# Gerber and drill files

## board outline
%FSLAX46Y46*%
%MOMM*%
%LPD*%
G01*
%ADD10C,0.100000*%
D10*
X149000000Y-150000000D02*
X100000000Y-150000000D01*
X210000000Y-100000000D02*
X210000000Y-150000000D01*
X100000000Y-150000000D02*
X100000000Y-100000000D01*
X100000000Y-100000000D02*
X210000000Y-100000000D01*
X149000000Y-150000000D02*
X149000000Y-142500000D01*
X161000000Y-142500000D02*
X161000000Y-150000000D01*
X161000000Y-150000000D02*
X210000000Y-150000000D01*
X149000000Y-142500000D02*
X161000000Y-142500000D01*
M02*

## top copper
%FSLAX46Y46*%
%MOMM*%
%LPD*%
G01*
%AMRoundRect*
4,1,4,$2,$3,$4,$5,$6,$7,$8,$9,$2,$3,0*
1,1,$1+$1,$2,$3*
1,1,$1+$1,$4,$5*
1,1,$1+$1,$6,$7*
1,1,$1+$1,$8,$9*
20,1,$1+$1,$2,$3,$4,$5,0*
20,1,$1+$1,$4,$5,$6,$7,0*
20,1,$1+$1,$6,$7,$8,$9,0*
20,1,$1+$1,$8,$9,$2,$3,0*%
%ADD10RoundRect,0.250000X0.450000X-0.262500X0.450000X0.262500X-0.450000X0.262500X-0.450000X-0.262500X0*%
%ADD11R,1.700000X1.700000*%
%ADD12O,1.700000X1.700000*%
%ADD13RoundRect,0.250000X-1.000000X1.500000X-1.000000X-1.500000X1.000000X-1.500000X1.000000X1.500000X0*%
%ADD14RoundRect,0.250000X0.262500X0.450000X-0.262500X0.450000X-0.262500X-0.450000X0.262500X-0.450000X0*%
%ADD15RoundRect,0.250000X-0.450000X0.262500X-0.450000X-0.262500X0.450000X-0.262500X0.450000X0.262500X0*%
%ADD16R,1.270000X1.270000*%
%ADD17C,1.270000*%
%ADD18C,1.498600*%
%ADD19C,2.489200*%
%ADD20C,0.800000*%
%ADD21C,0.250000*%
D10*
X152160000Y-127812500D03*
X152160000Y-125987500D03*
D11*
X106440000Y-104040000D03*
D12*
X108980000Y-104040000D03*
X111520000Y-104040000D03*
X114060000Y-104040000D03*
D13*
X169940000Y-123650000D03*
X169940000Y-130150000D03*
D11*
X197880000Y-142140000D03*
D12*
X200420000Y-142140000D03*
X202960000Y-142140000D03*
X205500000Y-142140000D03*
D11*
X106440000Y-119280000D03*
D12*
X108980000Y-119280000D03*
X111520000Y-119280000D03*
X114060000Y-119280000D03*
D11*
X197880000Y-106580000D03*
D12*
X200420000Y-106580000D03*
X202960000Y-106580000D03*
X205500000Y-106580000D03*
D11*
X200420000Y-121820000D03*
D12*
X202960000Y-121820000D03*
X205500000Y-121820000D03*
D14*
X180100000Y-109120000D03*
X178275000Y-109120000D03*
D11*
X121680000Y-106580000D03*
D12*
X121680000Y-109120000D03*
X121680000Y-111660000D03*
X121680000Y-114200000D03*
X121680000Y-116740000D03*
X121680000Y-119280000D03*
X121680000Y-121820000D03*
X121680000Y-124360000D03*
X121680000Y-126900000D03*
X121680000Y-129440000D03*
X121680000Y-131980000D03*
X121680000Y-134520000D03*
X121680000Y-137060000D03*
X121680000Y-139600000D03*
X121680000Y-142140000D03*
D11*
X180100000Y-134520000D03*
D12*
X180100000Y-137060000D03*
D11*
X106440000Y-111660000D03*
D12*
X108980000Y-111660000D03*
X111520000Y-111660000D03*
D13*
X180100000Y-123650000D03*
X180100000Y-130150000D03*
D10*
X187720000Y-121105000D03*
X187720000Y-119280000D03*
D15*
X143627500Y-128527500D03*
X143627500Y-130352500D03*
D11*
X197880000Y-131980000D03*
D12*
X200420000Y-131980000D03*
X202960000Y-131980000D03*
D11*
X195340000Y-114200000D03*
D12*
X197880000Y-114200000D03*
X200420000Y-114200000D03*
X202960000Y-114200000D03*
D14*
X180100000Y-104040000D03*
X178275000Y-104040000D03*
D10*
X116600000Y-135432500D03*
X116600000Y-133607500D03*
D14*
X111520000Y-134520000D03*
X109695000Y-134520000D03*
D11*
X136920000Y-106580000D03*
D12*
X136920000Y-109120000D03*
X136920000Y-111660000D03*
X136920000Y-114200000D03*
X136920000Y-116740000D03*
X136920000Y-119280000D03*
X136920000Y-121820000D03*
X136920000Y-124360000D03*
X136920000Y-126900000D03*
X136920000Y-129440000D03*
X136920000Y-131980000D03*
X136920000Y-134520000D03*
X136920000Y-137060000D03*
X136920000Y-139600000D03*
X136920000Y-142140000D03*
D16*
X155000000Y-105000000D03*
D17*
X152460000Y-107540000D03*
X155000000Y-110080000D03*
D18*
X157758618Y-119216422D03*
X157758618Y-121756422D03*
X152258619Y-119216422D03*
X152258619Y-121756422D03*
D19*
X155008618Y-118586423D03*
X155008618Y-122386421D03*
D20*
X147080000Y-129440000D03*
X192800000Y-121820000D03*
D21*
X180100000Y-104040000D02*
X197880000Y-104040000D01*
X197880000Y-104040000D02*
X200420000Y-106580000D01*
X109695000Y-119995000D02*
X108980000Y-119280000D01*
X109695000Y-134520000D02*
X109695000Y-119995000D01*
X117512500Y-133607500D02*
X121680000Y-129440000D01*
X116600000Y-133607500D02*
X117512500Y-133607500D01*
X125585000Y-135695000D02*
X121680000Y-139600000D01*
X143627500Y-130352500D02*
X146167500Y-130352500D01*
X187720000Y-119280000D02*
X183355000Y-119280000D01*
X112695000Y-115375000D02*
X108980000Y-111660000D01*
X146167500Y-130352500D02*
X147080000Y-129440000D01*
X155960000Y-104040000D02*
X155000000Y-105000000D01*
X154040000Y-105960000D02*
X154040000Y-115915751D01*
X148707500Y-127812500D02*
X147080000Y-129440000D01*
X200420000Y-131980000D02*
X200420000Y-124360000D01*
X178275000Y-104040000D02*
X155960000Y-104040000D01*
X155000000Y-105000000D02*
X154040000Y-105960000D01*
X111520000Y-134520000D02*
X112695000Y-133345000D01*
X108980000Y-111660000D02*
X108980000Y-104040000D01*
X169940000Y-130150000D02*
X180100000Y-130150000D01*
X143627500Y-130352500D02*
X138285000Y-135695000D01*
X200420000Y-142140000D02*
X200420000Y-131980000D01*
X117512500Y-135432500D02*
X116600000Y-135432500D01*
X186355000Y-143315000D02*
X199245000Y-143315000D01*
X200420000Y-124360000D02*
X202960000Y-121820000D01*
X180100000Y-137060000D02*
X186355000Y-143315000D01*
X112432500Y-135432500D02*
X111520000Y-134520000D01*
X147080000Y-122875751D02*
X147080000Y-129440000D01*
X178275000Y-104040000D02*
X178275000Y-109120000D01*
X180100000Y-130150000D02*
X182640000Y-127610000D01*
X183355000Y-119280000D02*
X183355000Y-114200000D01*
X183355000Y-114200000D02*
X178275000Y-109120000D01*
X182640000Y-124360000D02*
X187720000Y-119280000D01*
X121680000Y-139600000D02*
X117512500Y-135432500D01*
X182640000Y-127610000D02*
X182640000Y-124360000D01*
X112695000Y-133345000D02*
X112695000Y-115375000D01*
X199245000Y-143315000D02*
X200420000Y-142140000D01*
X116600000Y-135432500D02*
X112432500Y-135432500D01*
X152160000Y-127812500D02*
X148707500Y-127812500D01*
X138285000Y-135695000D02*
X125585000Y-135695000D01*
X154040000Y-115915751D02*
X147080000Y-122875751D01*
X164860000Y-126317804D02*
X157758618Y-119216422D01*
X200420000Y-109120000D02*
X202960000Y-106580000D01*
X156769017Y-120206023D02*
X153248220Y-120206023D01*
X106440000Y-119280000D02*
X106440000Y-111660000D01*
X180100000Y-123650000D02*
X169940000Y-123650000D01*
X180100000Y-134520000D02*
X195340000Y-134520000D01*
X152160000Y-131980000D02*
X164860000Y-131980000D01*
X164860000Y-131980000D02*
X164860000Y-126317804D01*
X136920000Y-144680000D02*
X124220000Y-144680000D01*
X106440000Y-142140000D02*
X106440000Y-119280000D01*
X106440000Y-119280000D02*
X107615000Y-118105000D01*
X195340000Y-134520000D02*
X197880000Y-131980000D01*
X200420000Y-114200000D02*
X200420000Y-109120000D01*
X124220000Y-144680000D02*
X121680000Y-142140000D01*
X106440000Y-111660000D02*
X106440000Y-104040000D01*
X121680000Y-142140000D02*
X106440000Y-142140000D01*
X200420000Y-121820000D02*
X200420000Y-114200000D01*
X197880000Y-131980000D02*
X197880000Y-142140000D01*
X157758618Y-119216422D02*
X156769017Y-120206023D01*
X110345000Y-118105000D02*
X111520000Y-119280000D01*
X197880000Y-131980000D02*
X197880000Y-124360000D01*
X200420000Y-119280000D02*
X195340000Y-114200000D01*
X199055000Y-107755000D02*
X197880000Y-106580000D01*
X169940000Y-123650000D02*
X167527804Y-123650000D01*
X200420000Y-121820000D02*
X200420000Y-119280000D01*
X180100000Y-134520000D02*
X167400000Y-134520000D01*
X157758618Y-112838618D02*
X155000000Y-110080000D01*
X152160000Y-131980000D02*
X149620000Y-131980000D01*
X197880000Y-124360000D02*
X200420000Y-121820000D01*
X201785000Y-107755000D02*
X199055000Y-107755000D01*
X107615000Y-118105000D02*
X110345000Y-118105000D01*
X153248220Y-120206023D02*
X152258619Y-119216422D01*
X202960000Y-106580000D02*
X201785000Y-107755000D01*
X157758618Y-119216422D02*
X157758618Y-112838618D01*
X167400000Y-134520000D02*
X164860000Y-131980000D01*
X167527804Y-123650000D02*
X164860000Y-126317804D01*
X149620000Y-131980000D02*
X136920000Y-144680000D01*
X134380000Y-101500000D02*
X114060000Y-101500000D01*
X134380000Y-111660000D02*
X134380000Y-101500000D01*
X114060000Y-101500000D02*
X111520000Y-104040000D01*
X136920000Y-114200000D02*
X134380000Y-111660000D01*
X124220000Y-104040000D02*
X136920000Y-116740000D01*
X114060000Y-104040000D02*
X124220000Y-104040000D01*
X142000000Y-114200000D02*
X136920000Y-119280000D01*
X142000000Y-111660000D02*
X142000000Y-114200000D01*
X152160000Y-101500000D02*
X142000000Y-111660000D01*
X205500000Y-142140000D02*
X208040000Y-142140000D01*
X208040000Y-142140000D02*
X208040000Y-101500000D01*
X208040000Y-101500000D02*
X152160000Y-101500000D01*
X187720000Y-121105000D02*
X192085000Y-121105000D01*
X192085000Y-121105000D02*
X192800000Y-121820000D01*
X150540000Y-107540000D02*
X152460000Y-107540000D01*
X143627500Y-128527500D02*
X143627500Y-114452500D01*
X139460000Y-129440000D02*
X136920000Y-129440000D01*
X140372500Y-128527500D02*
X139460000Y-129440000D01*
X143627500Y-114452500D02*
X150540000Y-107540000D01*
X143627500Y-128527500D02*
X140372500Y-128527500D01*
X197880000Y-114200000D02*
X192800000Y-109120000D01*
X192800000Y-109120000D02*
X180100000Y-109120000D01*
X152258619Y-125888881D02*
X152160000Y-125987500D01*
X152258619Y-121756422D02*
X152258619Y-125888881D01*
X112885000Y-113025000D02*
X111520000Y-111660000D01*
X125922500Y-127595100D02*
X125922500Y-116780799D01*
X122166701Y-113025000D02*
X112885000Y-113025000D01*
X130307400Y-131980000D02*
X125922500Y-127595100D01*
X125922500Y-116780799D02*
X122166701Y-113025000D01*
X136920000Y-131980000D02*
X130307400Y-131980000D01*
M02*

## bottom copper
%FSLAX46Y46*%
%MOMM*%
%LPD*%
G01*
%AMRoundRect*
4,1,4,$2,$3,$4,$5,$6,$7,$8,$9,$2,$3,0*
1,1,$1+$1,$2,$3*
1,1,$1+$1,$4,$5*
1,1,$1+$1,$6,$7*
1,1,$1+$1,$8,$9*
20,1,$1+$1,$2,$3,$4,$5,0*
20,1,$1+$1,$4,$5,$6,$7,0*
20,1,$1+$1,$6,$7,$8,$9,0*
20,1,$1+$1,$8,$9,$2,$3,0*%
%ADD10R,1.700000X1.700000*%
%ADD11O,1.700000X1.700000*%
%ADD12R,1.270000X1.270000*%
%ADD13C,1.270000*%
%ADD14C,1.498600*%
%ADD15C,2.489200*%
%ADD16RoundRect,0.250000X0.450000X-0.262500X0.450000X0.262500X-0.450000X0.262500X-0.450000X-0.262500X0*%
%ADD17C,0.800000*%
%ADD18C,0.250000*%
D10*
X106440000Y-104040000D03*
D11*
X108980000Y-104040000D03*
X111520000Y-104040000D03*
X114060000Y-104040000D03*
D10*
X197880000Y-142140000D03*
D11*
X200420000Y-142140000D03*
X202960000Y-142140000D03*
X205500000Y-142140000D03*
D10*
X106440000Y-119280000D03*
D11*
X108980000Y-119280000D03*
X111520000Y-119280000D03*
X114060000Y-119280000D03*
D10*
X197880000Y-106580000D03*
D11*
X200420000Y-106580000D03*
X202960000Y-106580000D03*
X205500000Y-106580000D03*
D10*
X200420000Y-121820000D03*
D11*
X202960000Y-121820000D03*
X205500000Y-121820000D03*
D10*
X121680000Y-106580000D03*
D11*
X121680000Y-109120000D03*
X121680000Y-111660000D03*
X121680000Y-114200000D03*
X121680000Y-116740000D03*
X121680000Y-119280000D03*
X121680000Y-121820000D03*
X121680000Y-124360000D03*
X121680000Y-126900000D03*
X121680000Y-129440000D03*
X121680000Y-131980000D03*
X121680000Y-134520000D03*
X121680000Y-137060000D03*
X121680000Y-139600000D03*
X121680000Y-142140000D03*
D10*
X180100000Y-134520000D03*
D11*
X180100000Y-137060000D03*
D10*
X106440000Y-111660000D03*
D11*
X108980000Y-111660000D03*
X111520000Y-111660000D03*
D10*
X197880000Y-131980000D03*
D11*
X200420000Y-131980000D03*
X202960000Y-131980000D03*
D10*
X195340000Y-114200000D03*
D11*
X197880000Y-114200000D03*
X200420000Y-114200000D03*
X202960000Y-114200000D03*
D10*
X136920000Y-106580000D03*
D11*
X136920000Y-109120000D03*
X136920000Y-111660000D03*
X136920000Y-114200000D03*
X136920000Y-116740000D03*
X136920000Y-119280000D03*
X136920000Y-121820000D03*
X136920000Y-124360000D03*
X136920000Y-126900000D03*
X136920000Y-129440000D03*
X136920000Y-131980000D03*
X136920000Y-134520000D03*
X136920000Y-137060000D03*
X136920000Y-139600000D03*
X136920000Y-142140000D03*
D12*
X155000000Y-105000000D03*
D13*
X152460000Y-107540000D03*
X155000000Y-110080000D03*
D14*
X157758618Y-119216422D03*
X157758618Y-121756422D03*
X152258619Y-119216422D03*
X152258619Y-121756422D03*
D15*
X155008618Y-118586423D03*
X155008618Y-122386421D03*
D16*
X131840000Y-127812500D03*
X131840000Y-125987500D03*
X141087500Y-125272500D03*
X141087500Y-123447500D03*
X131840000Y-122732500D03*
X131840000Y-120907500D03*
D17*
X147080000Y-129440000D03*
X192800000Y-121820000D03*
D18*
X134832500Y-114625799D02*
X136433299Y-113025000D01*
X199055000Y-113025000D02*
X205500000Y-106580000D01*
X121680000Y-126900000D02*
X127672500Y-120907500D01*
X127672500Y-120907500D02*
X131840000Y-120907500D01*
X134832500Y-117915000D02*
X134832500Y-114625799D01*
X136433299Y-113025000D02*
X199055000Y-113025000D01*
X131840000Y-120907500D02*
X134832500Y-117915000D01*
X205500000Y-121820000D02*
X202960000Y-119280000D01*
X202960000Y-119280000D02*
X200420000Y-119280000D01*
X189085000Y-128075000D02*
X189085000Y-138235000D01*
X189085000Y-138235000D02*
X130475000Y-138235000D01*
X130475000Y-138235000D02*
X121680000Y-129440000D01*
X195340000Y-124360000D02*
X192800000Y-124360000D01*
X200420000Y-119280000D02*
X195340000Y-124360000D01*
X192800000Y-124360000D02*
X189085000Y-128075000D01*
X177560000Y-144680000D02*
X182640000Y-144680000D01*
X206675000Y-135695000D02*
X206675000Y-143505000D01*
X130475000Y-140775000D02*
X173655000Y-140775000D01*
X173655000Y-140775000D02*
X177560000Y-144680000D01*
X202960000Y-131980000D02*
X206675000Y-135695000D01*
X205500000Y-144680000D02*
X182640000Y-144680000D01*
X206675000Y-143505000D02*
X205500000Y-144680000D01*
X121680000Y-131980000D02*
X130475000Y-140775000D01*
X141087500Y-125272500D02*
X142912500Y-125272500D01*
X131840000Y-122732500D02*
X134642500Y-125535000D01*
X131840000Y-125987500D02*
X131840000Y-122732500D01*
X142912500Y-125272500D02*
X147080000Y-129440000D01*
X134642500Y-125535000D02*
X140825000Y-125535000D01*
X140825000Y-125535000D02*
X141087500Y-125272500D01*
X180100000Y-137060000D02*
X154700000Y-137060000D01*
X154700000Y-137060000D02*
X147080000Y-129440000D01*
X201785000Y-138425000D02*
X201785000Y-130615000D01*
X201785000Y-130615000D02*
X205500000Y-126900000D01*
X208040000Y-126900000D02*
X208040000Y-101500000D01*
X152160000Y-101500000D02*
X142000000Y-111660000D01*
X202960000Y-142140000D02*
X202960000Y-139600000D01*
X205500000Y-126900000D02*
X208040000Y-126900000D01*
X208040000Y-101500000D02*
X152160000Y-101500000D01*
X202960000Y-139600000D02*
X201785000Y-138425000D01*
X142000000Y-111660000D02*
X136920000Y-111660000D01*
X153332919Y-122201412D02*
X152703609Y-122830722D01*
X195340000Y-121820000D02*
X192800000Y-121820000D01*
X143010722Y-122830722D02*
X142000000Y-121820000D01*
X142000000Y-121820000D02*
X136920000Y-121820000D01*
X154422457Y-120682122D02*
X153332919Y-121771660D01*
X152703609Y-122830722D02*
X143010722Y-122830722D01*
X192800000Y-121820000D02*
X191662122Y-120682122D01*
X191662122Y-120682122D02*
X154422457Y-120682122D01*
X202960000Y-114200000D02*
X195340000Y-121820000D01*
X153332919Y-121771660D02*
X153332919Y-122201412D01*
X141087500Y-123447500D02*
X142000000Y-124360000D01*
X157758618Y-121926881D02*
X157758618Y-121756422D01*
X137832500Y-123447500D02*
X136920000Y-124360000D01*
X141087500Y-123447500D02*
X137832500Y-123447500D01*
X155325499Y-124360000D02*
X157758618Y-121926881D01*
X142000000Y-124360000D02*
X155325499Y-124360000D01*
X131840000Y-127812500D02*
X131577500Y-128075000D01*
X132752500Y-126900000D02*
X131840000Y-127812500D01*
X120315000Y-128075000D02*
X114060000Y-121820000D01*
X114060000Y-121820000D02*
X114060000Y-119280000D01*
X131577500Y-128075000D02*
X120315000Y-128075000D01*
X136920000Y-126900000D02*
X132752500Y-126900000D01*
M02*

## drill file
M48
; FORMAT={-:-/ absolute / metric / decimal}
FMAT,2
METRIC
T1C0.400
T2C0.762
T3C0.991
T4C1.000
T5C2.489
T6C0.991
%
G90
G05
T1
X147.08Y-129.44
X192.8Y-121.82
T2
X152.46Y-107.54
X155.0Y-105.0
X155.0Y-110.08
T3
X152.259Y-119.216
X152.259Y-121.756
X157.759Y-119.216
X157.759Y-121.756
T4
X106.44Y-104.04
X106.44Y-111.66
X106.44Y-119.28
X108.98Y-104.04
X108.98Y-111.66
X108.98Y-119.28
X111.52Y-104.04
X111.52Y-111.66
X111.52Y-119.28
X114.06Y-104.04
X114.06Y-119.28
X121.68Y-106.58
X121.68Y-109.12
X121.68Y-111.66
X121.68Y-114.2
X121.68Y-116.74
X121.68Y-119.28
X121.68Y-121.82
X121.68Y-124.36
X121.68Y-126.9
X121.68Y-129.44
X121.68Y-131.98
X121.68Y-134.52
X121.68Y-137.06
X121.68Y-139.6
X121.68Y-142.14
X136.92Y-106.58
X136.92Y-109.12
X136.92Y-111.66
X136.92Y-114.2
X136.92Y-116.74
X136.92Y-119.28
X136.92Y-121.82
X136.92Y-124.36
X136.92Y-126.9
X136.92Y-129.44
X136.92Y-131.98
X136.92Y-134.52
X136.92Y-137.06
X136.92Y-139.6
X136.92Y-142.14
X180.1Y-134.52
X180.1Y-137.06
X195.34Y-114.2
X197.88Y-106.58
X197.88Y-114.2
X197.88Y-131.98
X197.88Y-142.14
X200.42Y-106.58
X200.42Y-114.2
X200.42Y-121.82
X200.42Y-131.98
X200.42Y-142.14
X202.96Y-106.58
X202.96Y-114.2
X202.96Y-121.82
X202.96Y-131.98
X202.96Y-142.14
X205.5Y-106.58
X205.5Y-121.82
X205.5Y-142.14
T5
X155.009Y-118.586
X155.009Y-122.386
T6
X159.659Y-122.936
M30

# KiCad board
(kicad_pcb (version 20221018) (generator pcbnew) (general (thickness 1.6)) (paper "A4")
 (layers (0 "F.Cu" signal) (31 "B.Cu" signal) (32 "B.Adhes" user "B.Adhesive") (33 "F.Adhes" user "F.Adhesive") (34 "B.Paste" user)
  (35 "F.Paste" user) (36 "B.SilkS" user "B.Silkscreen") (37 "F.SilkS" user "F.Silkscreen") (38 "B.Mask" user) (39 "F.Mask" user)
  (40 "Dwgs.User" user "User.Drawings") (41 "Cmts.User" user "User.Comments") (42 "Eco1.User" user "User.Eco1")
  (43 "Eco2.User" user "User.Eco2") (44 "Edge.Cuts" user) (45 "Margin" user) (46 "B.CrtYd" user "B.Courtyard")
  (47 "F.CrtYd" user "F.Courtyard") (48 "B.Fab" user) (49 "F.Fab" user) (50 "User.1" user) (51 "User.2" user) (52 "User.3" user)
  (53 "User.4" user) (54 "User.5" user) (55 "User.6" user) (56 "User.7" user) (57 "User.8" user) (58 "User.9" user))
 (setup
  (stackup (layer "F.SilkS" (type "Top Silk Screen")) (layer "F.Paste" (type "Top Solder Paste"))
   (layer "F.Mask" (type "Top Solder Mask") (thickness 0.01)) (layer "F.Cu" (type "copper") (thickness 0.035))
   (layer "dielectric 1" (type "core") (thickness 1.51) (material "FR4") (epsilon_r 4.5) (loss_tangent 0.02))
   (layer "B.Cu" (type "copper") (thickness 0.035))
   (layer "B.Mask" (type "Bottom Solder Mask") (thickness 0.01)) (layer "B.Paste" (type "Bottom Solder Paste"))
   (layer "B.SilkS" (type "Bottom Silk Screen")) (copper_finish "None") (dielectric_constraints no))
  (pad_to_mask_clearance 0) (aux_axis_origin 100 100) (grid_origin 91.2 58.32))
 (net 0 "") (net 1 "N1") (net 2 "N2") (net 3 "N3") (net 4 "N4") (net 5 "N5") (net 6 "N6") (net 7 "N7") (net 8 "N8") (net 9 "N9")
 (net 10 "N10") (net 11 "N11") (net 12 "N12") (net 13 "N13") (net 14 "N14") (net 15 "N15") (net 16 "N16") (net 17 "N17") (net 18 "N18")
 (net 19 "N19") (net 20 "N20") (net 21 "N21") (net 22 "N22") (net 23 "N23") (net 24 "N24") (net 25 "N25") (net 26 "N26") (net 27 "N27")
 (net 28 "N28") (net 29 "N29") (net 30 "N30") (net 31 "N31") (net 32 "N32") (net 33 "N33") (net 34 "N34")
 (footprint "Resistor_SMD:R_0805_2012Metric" (layer "F.Cu") (at 152.16 126.9 90)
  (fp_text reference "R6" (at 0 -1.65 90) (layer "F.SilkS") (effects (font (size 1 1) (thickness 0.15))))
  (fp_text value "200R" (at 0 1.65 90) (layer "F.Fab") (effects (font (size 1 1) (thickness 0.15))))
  (pad "1" smd roundrect (at -0.9125 0 90) (size 1.025 1.4) (layers "F.Cu" "F.Paste" "F.Mask") (roundrect_rratio 0.243902) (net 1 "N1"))
  (pad "2" smd roundrect (at 0.9125 0 90) (size 1.025 1.4) (layers "F.Cu" "F.Paste" "F.Mask") (roundrect_rratio 0.243902) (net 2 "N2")))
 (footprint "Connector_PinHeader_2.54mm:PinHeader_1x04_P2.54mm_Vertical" (layer "F.Cu") (at 106.44 104.04 90)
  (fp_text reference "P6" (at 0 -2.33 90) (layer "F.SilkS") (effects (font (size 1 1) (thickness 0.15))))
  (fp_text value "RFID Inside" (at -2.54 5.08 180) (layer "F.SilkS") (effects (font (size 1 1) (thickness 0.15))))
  (pad "1" thru_hole rect (at 0 0 90) (size 1.7 1.7) (drill 1) (layers "*.Cu" "*.Mask") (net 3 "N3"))
  (pad "2" thru_hole oval (at 0 2.54 90) (size 1.7 1.7) (drill 1) (layers "*.Cu" "*.Mask") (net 1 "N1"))
  (pad "3" thru_hole oval (at 0 5.08 90) (size 1.7 1.7) (drill 1) (layers "*.Cu" "*.Mask") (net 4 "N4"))
  (pad "4" thru_hole oval (at 0 7.62 90) (size 1.7 1.7) (drill 1) (layers "*.Cu" "*.Mask") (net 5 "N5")))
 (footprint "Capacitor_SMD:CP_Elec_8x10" (layer "F.Cu") (at 169.94 126.9 -90)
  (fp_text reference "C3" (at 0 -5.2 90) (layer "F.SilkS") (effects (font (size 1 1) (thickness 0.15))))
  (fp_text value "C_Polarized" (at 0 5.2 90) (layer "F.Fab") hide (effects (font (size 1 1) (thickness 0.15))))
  (pad "1" smd roundrect (at -3.25 0 270) (size 3.5 2.5) (layers "F.Cu" "F.Paste" "F.Mask") (roundrect_rratio 0.1) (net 3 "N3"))
  (pad "2" smd roundrect (at 3.25 0 270) (size 3.5 2.5) (layers "F.Cu" "F.Paste" "F.Mask") (roundrect_rratio 0.1) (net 1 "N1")))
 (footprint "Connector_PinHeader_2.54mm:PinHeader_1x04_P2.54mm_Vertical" (layer "F.Cu") (at 197.88 142.14 90)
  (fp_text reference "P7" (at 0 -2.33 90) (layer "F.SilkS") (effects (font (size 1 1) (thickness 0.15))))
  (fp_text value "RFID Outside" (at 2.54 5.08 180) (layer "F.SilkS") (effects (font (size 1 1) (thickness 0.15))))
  (pad "1" thru_hole rect (at 0 0 90) (size 1.7 1.7) (drill 1) (layers "*.Cu" "*.Mask") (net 3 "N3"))
  (pad "2" thru_hole oval (at 0 2.54 90) (size 1.7 1.7) (drill 1) (layers "*.Cu" "*.Mask") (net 1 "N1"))
  (pad "3" thru_hole oval (at 0 5.08 90) (size 1.7 1.7) (drill 1) (layers "*.Cu" "*.Mask") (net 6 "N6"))
  (pad "4" thru_hole oval (at 0 7.62 90) (size 1.7 1.7) (drill 1) (layers "*.Cu" "*.Mask") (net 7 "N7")))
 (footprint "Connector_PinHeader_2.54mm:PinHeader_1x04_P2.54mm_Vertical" (layer "F.Cu") (at 106.44 119.28 90)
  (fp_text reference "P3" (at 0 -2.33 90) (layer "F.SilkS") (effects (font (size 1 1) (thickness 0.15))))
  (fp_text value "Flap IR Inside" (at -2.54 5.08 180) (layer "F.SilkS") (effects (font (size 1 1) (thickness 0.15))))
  (pad "1" thru_hole rect (at 0 0 90) (size 1.7 1.7) (drill 1) (layers "*.Cu" "*.Mask") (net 3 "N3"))
  (pad "2" thru_hole oval (at 0 2.54 90) (size 1.7 1.7) (drill 1) (layers "*.Cu" "*.Mask") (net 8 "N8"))
  (pad "3" thru_hole oval (at 0 5.08 90) (size 1.7 1.7) (drill 1) (layers "*.Cu" "*.Mask") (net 3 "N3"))
  (pad "4" thru_hole oval (at 0 7.62 90) (size 1.7 1.7) (drill 1) (layers "*.Cu" "*.Mask") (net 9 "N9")))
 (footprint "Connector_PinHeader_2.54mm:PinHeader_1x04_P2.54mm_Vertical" (layer "F.Cu") (at 197.88 106.58 90)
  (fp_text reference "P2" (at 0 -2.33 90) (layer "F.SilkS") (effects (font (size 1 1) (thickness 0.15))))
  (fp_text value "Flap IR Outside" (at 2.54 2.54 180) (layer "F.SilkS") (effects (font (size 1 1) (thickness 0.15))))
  (pad "1" thru_hole rect (at 0 0 90) (size 1.7 1.7) (drill 1) (layers "*.Cu" "*.Mask") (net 3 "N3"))
  (pad "2" thru_hole oval (at 0 2.54 90) (size 1.7 1.7) (drill 1) (layers "*.Cu" "*.Mask") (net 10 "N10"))
  (pad "3" thru_hole oval (at 0 5.08 90) (size 1.7 1.7) (drill 1) (layers "*.Cu" "*.Mask") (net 3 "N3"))
  (pad "4" thru_hole oval (at 0 7.62 90) (size 1.7 1.7) (drill 1) (layers "*.Cu" "*.Mask") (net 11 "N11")))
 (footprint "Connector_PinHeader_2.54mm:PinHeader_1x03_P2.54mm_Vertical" (layer "F.Cu") (at 200.42 121.82 90)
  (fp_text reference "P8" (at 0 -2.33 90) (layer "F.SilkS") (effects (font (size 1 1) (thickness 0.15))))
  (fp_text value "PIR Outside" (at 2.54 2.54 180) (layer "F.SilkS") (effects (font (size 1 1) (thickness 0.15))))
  (pad "1" thru_hole rect (at 0 0 90) (size 1.7 1.7) (drill 1) (layers "*.Cu" "*.Mask") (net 3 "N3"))
  (pad "2" thru_hole oval (at 0 2.54 90) (size 1.7 1.7) (drill 1) (layers "*.Cu" "*.Mask") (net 1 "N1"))
  (pad "3" thru_hole oval (at 0 5.08 90) (size 1.7 1.7) (drill 1) (layers "*.Cu" "*.Mask") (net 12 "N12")))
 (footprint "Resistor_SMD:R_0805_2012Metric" (layer "F.Cu") (at 179.1875 109.12 180)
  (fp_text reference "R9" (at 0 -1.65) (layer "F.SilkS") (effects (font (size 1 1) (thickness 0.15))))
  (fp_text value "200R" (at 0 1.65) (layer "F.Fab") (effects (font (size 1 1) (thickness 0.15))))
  (pad "1" smd roundrect (at -0.9125 0 180) (size 1.025 1.4) (layers "F.Cu" "F.Paste" "F.Mask") (roundrect_rratio 0.243902) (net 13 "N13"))
  (pad "2" smd roundrect (at 0.9125 0 180) (size 1.025 1.4) (layers "F.Cu" "F.Paste" "F.Mask") (roundrect_rratio 0.243902) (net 1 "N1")))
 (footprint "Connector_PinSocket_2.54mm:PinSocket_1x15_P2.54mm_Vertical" (layer "F.Cu") (at 121.68 106.58)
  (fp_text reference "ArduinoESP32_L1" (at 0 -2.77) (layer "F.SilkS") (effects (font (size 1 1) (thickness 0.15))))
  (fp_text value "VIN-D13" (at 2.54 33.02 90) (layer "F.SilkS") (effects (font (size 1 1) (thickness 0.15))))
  (pad "1" thru_hole rect (at 0 0) (size 1.7 1.7) (drill 1) (layers "*.Cu" "*.Mask") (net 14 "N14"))
  (pad "2" thru_hole oval (at 0 2.54) (size 1.7 1.7) (drill 1) (layers "*.Cu" "*.Mask") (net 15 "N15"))
  (pad "3" thru_hole oval (at 0 5.08) (size 1.7 1.7) (drill 1) (layers "*.Cu" "*.Mask") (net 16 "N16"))
  (pad "4" thru_hole oval (at 0 7.62) (size 1.7 1.7) (drill 1) (layers "*.Cu" "*.Mask") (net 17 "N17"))
  (pad "5" thru_hole oval (at 0 10.16) (size 1.7 1.7) (drill 1) (layers "*.Cu" "*.Mask") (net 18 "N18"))
  (pad "6" thru_hole oval (at 0 12.7) (size 1.7 1.7) (drill 1) (layers "*.Cu" "*.Mask") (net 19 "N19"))
  (pad "7" thru_hole oval (at 0 15.24) (size 1.7 1.7) (drill 1) (layers "*.Cu" "*.Mask") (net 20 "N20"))
  (pad "8" thru_hole oval (at 0 17.78) (size 1.7 1.7) (drill 1) (layers "*.Cu" "*.Mask") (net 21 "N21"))
  (pad "9" thru_hole oval (at 0 20.32) (size 1.7 1.7) (drill 1) (layers "*.Cu" "*.Mask") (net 11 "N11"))
  (pad "10" thru_hole oval (at 0 22.86) (size 1.7 1.7) (drill 1) (layers "*.Cu" "*.Mask") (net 12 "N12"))
  (pad "11" thru_hole oval (at 0 25.4) (size 1.7 1.7) (drill 1) (layers "*.Cu" "*.Mask") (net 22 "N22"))
  (pad "12" thru_hole oval (at 0 27.94) (size 1.7 1.7) (drill 1) (layers "*.Cu" "*.Mask") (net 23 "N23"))
  (pad "13" thru_hole oval (at 0 30.48) (size 1.7 1.7) (drill 1) (layers "*.Cu" "*.Mask") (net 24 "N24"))
  (pad "14" thru_hole oval (at 0 33.02) (size 1.7 1.7) (drill 1) (layers "*.Cu" "*.Mask") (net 1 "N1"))
  (pad "15" thru_hole oval (at 0 35.56) (size 1.7 1.7) (drill 1) (layers "*.Cu" "*.Mask") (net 3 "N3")))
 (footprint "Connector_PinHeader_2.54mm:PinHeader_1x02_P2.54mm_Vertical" (layer "F.Cu") (at 180.1 134.52)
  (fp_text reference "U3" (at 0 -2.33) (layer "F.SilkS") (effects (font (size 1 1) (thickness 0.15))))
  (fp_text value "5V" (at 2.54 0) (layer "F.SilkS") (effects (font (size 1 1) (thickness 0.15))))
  (pad "1" thru_hole rect (at 0 0) (size 1.7 1.7) (drill 1) (layers "*.Cu" "*.Mask") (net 3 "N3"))
  (pad "2" thru_hole oval (at 0 2.54) (size 1.7 1.7) (drill 1) (layers "*.Cu" "*.Mask") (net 1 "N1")))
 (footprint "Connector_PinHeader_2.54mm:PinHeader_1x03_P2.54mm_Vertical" (layer "F.Cu") (at 106.44 111.66 90)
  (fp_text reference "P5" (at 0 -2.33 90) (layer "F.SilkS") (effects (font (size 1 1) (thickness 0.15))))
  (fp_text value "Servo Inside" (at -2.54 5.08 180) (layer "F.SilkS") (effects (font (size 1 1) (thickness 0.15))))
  (pad "1" thru_hole rect (at 0 0 90) (size 1.7 1.7) (drill 1) (layers "*.Cu" "*.Mask") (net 3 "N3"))
  (pad "2" thru_hole oval (at 0 2.54 90) (size 1.7 1.7) (drill 1) (layers "*.Cu" "*.Mask") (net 1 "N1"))
  (pad "3" thru_hole oval (at 0 5.08 90) (size 1.7 1.7) (drill 1) (layers "*.Cu" "*.Mask") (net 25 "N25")))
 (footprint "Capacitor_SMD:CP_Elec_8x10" (layer "F.Cu") (at 180.1 126.9 -90)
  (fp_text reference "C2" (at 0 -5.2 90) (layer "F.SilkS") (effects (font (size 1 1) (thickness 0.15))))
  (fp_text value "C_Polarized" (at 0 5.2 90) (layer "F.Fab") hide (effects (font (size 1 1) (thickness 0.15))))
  (pad "1" smd roundrect (at -3.25 0 270) (size 3.5 2.5) (layers "F.Cu" "F.Paste" "F.Mask") (roundrect_rratio 0.1) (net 3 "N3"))
  (pad "2" smd roundrect (at 3.25 0 270) (size 3.5 2.5) (layers "F.Cu" "F.Paste" "F.Mask") (roundrect_rratio 0.1) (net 1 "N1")))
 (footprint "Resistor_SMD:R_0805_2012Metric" (layer "F.Cu") (at 187.72 120.1925 90)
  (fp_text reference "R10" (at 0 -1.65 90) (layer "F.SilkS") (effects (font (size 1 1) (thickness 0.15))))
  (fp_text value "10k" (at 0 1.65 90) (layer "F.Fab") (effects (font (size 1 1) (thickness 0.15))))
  (pad "1" smd roundrect (at -0.9125 0 90) (size 1.025 1.4) (layers "F.Cu" "F.Paste" "F.Mask") (roundrect_rratio 0.243902) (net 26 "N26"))
  (pad "2" smd roundrect (at 0.9125 0 90) (size 1.025 1.4) (layers "F.Cu" "F.Paste" "F.Mask") (roundrect_rratio 0.243902) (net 1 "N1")))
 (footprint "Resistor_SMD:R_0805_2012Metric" (layer "F.Cu") (at 143.6275 129.44 -90)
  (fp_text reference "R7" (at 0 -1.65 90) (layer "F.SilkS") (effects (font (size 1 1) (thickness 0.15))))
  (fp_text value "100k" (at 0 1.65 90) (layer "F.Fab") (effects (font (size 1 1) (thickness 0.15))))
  (pad "1" smd roundrect (at -0.9125 0 270) (size 1.025 1.4) (layers "F.Cu" "F.Paste" "F.Mask") (roundrect_rratio 0.243902) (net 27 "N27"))
  (pad "2" smd roundrect (at 0.9125 0 270) (size 1.025 1.4) (layers "F.Cu" "F.Paste" "F.Mask") (roundrect_rratio 0.243902) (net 1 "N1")))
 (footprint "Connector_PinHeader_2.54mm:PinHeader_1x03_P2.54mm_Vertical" (layer "F.Cu") (at 197.88 131.98 90)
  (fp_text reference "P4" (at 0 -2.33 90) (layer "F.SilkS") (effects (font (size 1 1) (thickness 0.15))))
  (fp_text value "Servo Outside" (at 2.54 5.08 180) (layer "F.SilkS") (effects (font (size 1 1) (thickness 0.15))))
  (pad "1" thru_hole rect (at 0 0 90) (size 1.7 1.7) (drill 1) (layers "*.Cu" "*.Mask") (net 3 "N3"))
  (pad "2" thru_hole oval (at 0 2.54 90) (size 1.7 1.7) (drill 1) (layers "*.Cu" "*.Mask") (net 1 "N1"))
  (pad "3" thru_hole oval (at 0 5.08 90) (size 1.7 1.7) (drill 1) (layers "*.Cu" "*.Mask") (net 22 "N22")))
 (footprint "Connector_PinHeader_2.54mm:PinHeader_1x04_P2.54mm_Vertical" (layer "F.Cu") (at 195.34 114.2 90)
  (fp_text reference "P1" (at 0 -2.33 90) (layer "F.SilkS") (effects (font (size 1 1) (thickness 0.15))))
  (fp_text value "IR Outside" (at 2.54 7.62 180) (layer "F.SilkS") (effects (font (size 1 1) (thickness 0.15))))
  (pad "1" thru_hole rect (at 0 0 90) (size 1.7 1.7) (drill 1) (layers "*.Cu" "*.Mask") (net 3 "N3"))
  (pad "2" thru_hole oval (at 0 2.54 90) (size 1.7 1.7) (drill 1) (layers "*.Cu" "*.Mask") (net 13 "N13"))
  (pad "3" thru_hole oval (at 0 5.08 90) (size 1.7 1.7) (drill 1) (layers "*.Cu" "*.Mask") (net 3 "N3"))
  (pad "4" thru_hole oval (at 0 7.62 90) (size 1.7 1.7) (drill 1) (layers "*.Cu" "*.Mask") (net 26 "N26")))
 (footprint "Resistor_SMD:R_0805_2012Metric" (layer "F.Cu") (at 179.1875 104.04 180)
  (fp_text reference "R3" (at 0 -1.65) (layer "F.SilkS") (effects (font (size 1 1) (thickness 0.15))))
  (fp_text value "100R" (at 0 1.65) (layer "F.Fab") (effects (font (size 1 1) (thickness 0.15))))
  (pad "1" smd roundrect (at -0.9125 0 180) (size 1.025 1.4) (layers "F.Cu" "F.Paste" "F.Mask") (roundrect_rratio 0.243902) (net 10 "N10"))
  (pad "2" smd roundrect (at 0.9125 0 180) (size 1.025 1.4) (layers "F.Cu" "F.Paste" "F.Mask") (roundrect_rratio 0.243902) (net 1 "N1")))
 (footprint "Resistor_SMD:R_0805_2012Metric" (layer "F.Cu") (at 116.6 134.52 90)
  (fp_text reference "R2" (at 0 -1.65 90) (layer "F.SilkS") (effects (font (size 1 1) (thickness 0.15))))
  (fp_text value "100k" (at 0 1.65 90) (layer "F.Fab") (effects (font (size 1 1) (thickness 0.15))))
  (pad "1" smd roundrect (at -0.9125 0 90) (size 1.025 1.4) (layers "F.Cu" "F.Paste" "F.Mask") (roundrect_rratio 0.243902) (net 1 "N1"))
  (pad "2" smd roundrect (at 0.9125 0 90) (size 1.025 1.4) (layers "F.Cu" "F.Paste" "F.Mask") (roundrect_rratio 0.243902) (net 12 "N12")))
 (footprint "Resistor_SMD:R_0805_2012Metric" (layer "F.Cu") (at 110.6075 134.52 180)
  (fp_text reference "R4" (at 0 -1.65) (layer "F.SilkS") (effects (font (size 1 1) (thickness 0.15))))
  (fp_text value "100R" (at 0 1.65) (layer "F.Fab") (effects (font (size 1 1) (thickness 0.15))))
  (pad "1" smd roundrect (at -0.9125 0 180) (size 1.025 1.4) (layers "F.Cu" "F.Paste" "F.Mask") (roundrect_rratio 0.243902) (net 1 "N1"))
  (pad "2" smd roundrect (at 0.9125 0 180) (size 1.025 1.4) (layers "F.Cu" "F.Paste" "F.Mask") (roundrect_rratio 0.243902) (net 8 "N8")))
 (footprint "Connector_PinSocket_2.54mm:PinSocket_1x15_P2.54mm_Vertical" (layer "F.Cu") (at 136.92 106.58)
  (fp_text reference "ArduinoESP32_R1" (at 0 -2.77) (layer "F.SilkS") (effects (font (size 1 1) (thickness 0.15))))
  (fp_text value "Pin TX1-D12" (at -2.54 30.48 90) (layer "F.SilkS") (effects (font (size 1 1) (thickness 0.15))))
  (pad "1" thru_hole rect (at 0 0) (size 1.7 1.7) (drill 1) (layers "*.Cu" "*.Mask") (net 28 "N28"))
  (pad "2" thru_hole oval (at 0 2.54) (size 1.7 1.7) (drill 1) (layers "*.Cu" "*.Mask") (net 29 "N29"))
  (pad "3" thru_hole oval (at 0 5.08) (size 1.7 1.7) (drill 1) (layers "*.Cu" "*.Mask") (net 6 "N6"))
  (pad "4" thru_hole oval (at 0 7.62) (size 1.7 1.7) (drill 1) (layers "*.Cu" "*.Mask") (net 4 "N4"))
  (pad "5" thru_hole oval (at 0 10.16) (size 1.7 1.7) (drill 1) (layers "*.Cu" "*.Mask") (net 5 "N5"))
  (pad "6" thru_hole oval (at 0 12.7) (size 1.7 1.7) (drill 1) (layers "*.Cu" "*.Mask") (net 7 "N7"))
  (pad "7" thru_hole oval (at 0 15.24) (size 1.7 1.7) (drill 1) (layers "*.Cu" "*.Mask") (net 26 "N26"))
  (pad "8" thru_hole oval (at 0 17.78) (size 1.7 1.7) (drill 1) (layers "*.Cu" "*.Mask") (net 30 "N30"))
  (pad "9" thru_hole oval (at 0 20.32) (size 1.7 1.7) (drill 1) (layers "*.Cu" "*.Mask") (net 9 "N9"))
  (pad "10" thru_hole oval (at 0 22.86) (size 1.7 1.7) (drill 1) (layers "*.Cu" "*.Mask") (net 27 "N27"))
  (pad "11" thru_hole oval (at 0 25.4) (size 1.7 1.7) (drill 1) (layers "*.Cu" "*.Mask") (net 25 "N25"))
  (pad "12" thru_hole oval (at 0 27.94) (size 1.7 1.7) (drill 1) (layers "*.Cu" "*.Mask") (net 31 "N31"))
  (pad "13" thru_hole oval (at 0 30.48) (size 1.7 1.7) (drill 1) (layers "*.Cu" "*.Mask") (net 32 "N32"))
  (pad "14" thru_hole oval (at 0 33.02) (size 1.7 1.7) (drill 1) (layers "*.Cu" "*.Mask") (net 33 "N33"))
  (pad "15" thru_hole oval (at 0 35.56) (size 1.7 1.7) (drill 1) (layers "*.Cu" "*.Mask") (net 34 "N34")))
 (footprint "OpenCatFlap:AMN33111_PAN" (layer "B.Cu") (at 155 105 180)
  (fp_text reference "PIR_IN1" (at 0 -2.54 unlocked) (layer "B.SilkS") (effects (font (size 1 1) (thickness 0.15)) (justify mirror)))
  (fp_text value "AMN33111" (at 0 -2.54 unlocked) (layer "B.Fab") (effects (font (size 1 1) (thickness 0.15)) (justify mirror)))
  (pad "1" thru_hole rect (at 0 0 180) (size 1.27 1.27) (drill 0.762) (layers "*.Cu" "*.Mask") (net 1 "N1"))
  (pad "2" thru_hole circle (at 2.54 -2.54 90) (size 1.27 1.27) (drill 0.762) (layers "*.Cu" "*.Mask") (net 27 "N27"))
  (pad "3" thru_hole circle (at 0 -5.08 180) (size 1.27 1.27) (drill 0.762) (layers "*.Cu" "*.Mask") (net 3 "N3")))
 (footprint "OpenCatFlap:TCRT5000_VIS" (layer "B.Cu") (at 157.758618 119.216422 180)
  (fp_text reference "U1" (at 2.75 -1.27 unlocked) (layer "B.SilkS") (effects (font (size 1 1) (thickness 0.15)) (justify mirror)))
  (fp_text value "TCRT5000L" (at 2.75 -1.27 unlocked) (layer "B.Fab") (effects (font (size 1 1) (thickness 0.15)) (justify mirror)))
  (pad "" np_thru_hole circle (at -1.900001 -3.72 180) (size 0.9906 0.9906) (drill 0.9906) (layers "*.Cu" "*.Mask"))
  (pad "1" thru_hole circle (at 0 0 180) (size 1.4986 1.4986) (drill 0.9906) (layers "*.Cu" "*.Mask") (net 3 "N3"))
  (pad "2" thru_hole circle (at 0 -2.54 180) (size 1.4986 1.4986) (drill 0.9906) (layers "*.Cu" "*.Mask") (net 30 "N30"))
  (pad "3" thru_hole circle (at 5.499999 0 180) (size 1.4986 1.4986) (drill 0.9906) (layers "*.Cu" "*.Mask") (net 3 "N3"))
  (pad "4" thru_hole circle (at 5.499999 -2.54 180) (size 1.4986 1.4986) (drill 0.9906) (layers "*.Cu" "*.Mask") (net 2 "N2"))
  (pad "5" thru_hole circle (at 2.75 0.629999 180) (size 2.4892 2.4892) (drill 2.4892) (layers "*.Cu" "*.Mask"))
  (pad "6" thru_hole circle (at 2.75 -3.169999 180) (size 2.4892 2.4892) (drill 2.4892) (layers "*.Cu" "*.Mask")))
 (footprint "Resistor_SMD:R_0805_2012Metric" (layer "B.Cu") (at 131.84 126.9 90)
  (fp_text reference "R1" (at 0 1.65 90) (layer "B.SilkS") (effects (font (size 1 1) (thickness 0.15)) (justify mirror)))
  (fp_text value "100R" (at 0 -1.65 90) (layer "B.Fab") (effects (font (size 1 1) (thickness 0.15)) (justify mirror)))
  (pad "1" smd roundrect (at -0.9125 0 90) (size 1.025 1.4) (layers "B.Cu" "B.Paste" "B.Mask") (roundrect_rratio 0.243902) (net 9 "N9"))
  (pad "2" smd roundrect (at 0.9125 0 90) (size 1.025 1.4) (layers "B.Cu" "B.Paste" "B.Mask") (roundrect_rratio 0.243902) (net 1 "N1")))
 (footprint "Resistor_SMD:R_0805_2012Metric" (layer "B.Cu") (at 141.0875 124.36 90)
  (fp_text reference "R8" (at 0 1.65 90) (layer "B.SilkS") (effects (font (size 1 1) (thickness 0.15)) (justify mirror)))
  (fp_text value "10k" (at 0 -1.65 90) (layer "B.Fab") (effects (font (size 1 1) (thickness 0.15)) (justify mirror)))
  (pad "1" smd roundrect (at -0.9125 0 90) (size 1.025 1.4) (layers "B.Cu" "B.Paste" "B.Mask") (roundrect_rratio 0.243902) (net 1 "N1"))
  (pad "2" smd roundrect (at 0.9125 0 90) (size 1.025 1.4) (layers "B.Cu" "B.Paste" "B.Mask") (roundrect_rratio 0.243902) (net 30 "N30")))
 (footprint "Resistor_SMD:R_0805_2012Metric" (layer "B.Cu") (at 131.84 121.82 90)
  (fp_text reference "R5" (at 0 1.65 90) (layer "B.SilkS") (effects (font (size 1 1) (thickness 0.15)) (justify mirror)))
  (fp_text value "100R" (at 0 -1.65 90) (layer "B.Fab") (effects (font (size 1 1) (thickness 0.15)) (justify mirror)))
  (pad "1" smd roundrect (at -0.9125 0 90) (size 1.025 1.4) (layers "B.Cu" "B.Paste" "B.Mask") (roundrect_rratio 0.243902) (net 1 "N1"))
  (pad "2" smd roundrect (at 0.9125 0 90) (size 1.025 1.4) (layers "B.Cu" "B.Paste" "B.Mask") (roundrect_rratio 0.243902) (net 11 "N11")))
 (gr_line (start 149 150) (end 100 150) (stroke (width 0.1) (type default)) (layer "Edge.Cuts"))
 (gr_line locked (start 210 100) (end 210 150) (stroke (width 0.1) (type default)) (layer "Edge.Cuts"))
 (gr_line locked (start 100 150) (end 100 100) (stroke (width 0.1) (type default)) (layer "Edge.Cuts"))
 (gr_line locked (start 100 100) (end 210 100) (stroke (width 0.1) (type default)) (layer "Edge.Cuts"))
 (gr_line (start 149 150) (end 149 142.5) (stroke (width 0.1) (type default)) (layer "Edge.Cuts"))
 (gr_line (start 161 142.5) (end 161 150) (stroke (width 0.1) (type default)) (layer "Edge.Cuts"))
 (gr_line (start 161 150) (end 210 150) (stroke (width 0.1) (type default)) (layer "Edge.Cuts"))
 (gr_line (start 149 142.5) (end 161 142.5) (stroke (width 0.1) (type default)) (layer "Edge.Cuts"))
 (segment (start 180.1 104.04) (end 197.88 104.04) (width 0.25) (layer "F.Cu") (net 10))
 (segment (start 197.88 104.04) (end 200.42 106.58) (width 0.25) (layer "F.Cu") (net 10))
 (segment (start 109.695 119.995) (end 108.98 119.28) (width 0.25) (layer "F.Cu") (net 8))
 (segment (start 109.695 134.52) (end 109.695 119.995) (width 0.25) (layer "F.Cu") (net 8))
 (segment (start 134.8325 114.625799) (end 136.433299 113.025) (width 0.25) (layer "B.Cu") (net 11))
 (segment (start 199.055 113.025) (end 205.5 106.58) (width 0.25) (layer "B.Cu") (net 11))
 (segment (start 121.68 126.9) (end 127.6725 120.9075) (width 0.25) (layer "B.Cu") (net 11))
 (segment (start 127.6725 120.9075) (end 131.84 120.9075) (width 0.25) (layer "B.Cu") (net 11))
 (segment (start 134.8325 117.915) (end 134.8325 114.625799) (width 0.25) (layer "B.Cu") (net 11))
 (segment (start 136.433299 113.025) (end 199.055 113.025) (width 0.25) (layer "B.Cu") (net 11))
 (segment (start 131.84 120.9075) (end 134.8325 117.915) (width 0.25) (layer "B.Cu") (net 11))
 (segment (start 117.5125 133.6075) (end 121.68 129.44) (width 0.25) (layer "F.Cu") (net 12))
 (segment (start 116.6 133.6075) (end 117.5125 133.6075) (width 0.25) (layer "F.Cu") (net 12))
 (segment (start 205.5 121.82) (end 202.96 119.28) (width 0.25) (layer "B.Cu") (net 12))
 (segment (start 202.96 119.28) (end 200.42 119.28) (width 0.25) (layer "B.Cu") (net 12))
 (segment (start 189.085 128.075) (end 189.085 138.235) (width 0.25) (layer "B.Cu") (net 12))
 (segment (start 189.085 138.235) (end 130.475 138.235) (width 0.25) (layer "B.Cu") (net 12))
 (segment (start 130.475 138.235) (end 121.68 129.44) (width 0.25) (layer "B.Cu") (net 12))
 (segment (start 195.34 124.36) (end 192.8 124.36) (width 0.25) (layer "B.Cu") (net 12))
 (segment (start 200.42 119.28) (end 195.34 124.36) (width 0.25) (layer "B.Cu") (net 12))
 (segment (start 192.8 124.36) (end 189.085 128.075) (width 0.25) (layer "B.Cu") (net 12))
 (segment (start 177.56 144.68) (end 182.64 144.68) (width 0.25) (layer "B.Cu") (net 22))
 (segment (start 206.675 135.695) (end 206.675 143.505) (width 0.25) (layer "B.Cu") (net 22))
 (segment (start 130.475 140.775) (end 173.655 140.775) (width 0.25) (layer "B.Cu") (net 22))
 (segment (start 173.655 140.775) (end 177.56 144.68) (width 0.25) (layer "B.Cu") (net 22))
 (segment (start 202.96 131.98) (end 206.675 135.695) (width 0.25) (layer "B.Cu") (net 22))
 (segment (start 205.5 144.68) (end 182.64 144.68) (width 0.25) (layer "B.Cu") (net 22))
 (segment (start 206.675 143.505) (end 205.5 144.68) (width 0.25) (layer "B.Cu") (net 22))
 (segment (start 121.68 131.98) (end 130.475 140.775) (width 0.25) (layer "B.Cu") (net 22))
 (segment (start 125.585 135.695) (end 121.68 139.6) (width 0.25) (layer "F.Cu") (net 1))
 (segment (start 143.6275 130.3525) (end 146.1675 130.3525) (width 0.25) (layer "F.Cu") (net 1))
 (segment (start 187.72 119.28) (end 183.355 119.28) (width 0.25) (layer "F.Cu") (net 1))
 (segment (start 112.695 115.375) (end 108.98 111.66) (width 0.25) (layer "F.Cu") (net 1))
 (segment (start 146.1675 130.3525) (end 147.08 129.44) (width 0.25) (layer "F.Cu") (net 1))
 (segment (start 155.96 104.04) (end 155 105) (width 0.25) (layer "F.Cu") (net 1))
 (segment (start 154.04 105.96) (end 154.04 115.915751) (width 0.25) (layer "F.Cu") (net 1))
 (segment (start 148.7075 127.8125) (end 147.08 129.44) (width 0.25) (layer "F.Cu") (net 1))
 (segment (start 200.42 131.98) (end 200.42 124.36) (width 0.25) (layer "F.Cu") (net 1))
 (segment (start 178.275 104.04) (end 155.96 104.04) (width 0.25) (layer "F.Cu") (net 1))
 (segment (start 155 105) (end 154.04 105.96) (width 0.25) (layer "F.Cu") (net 1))
 (segment (start 111.52 134.52) (end 112.695 133.345) (width 0.25) (layer "F.Cu") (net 1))
 (segment (start 108.98 111.66) (end 108.98 104.04) (width 0.25) (layer "F.Cu") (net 1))
 (segment (start 169.94 130.15) (end 180.1 130.15) (width 0.25) (layer "F.Cu") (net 1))
 (segment (start 143.6275 130.3525) (end 138.285 135.695) (width 0.25) (layer "F.Cu") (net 1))
 (segment (start 200.42 142.14) (end 200.42 131.98) (width 0.25) (layer "F.Cu") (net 1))
 (segment (start 117.5125 135.4325) (end 116.6 135.4325) (width 0.25) (layer "F.Cu") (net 1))
 (segment (start 186.355 143.315) (end 199.245 143.315) (width 0.25) (layer "F.Cu") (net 1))
 (segment (start 200.42 124.36) (end 202.96 121.82) (width 0.25) (layer "F.Cu") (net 1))
 (segment (start 180.1 137.06) (end 186.355 143.315) (width 0.25) (layer "F.Cu") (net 1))
 (segment (start 112.4325 135.4325) (end 111.52 134.52) (width 0.25) (layer "F.Cu") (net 1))
 (segment (start 147.08 122.875751) (end 147.08 129.44) (width 0.25) (layer "F.Cu") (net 1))
 (segment (start 178.275 104.04) (end 178.275 109.12) (width 0.25) (layer "F.Cu") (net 1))
 (segment (start 180.1 130.15) (end 182.64 127.61) (width 0.25) (layer "F.Cu") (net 1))
 (segment (start 183.355 119.28) (end 183.355 114.2) (width 0.25) (layer "F.Cu") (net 1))
 (segment (start 183.355 114.2) (end 178.275 109.12) (width 0.25) (layer "F.Cu") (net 1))
 (segment (start 182.64 124.36) (end 187.72 119.28) (width 0.25) (layer "F.Cu") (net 1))
 (segment (start 121.68 139.6) (end 117.5125 135.4325) (width 0.25) (layer "F.Cu") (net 1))
 (segment (start 182.64 127.61) (end 182.64 124.36) (width 0.25) (layer "F.Cu") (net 1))
 (segment (start 112.695 133.345) (end 112.695 115.375) (width 0.25) (layer "F.Cu") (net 1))
 (segment (start 199.245 143.315) (end 200.42 142.14) (width 0.25) (layer "F.Cu") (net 1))
 (segment (start 116.6 135.4325) (end 112.4325 135.4325) (width 0.25) (layer "F.Cu") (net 1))
 (segment (start 152.16 127.8125) (end 148.7075 127.8125) (width 0.25) (layer "F.Cu") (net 1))
 (segment (start 138.285 135.695) (end 125.585 135.695) (width 0.25) (layer "F.Cu") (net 1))
 (segment (start 154.04 115.915751) (end 147.08 122.875751) (width 0.25) (layer "F.Cu") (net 1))
 (via blind (at 147.08 129.44) (size 0.8) (drill 0.4) (layers "F.Cu" "B.Cu") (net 1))
 (segment (start 141.0875 125.2725) (end 142.9125 125.2725) (width 0.25) (layer "B.Cu") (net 1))
 (segment (start 131.84 122.7325) (end 134.6425 125.535) (width 0.25) (layer "B.Cu") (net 1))
 (segment (start 131.84 125.9875) (end 131.84 122.7325) (width 0.25) (layer "B.Cu") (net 1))
 (segment (start 142.9125 125.2725) (end 147.08 129.44) (width 0.25) (layer "B.Cu") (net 1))
 (segment (start 134.6425 125.535) (end 140.825 125.535) (width 0.25) (layer "B.Cu") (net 1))
 (segment (start 140.825 125.535) (end 141.0875 125.2725) (width 0.25) (layer "B.Cu") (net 1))
 (segment (start 180.1 137.06) (end 154.7 137.06) (width 0.25) (layer "B.Cu") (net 1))
 (segment (start 154.7 137.06) (end 147.08 129.44) (width 0.25) (layer "B.Cu") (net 1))
 (segment (start 164.86 126.317804) (end 157.758618 119.216422) (width 0.25) (layer "F.Cu") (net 3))
 (segment (start 200.42 109.12) (end 202.96 106.58) (width 0.25) (layer "F.Cu") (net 3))
 (segment (start 156.769017 120.206023) (end 153.24822 120.206023) (width 0.25) (layer "F.Cu") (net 3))
 (segment (start 106.44 119.28) (end 106.44 111.66) (width 0.25) (layer "F.Cu") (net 3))
 (segment (start 180.1 123.65) (end 169.94 123.65) (width 0.25) (layer "F.Cu") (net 3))
 (segment (start 180.1 134.52) (end 195.34 134.52) (width 0.25) (layer "F.Cu") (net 3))
 (segment (start 152.16 131.98) (end 164.86 131.98) (width 0.25) (layer "F.Cu") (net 3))
 (segment (start 164.86 131.98) (end 164.86 126.317804) (width 0.25) (layer "F.Cu") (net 3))
 (segment (start 136.92 144.68) (end 124.22 144.68) (width 0.25) (layer "F.Cu") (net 3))
 (segment (start 106.44 142.14) (end 106.44 119.28) (width 0.25) (layer "F.Cu") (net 3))
 (segment (start 106.44 119.28) (end 107.615 118.105) (width 0.25) (layer "F.Cu") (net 3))
 (segment (start 195.34 134.52) (end 197.88 131.98) (width 0.25) (layer "F.Cu") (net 3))
 (segment (start 200.42 114.2) (end 200.42 109.12) (width 0.25) (layer "F.Cu") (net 3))
 (segment (start 124.22 144.68) (end 121.68 142.14) (width 0.25) (layer "F.Cu") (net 3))
 (segment (start 106.44 111.66) (end 106.44 104.04) (width 0.25) (layer "F.Cu") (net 3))
 (segment (start 121.68 142.14) (end 106.44 142.14) (width 0.25) (layer "F.Cu") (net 3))
 (segment (start 200.42 121.82) (end 200.42 114.2) (width 0.25) (layer "F.Cu") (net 3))
 (segment (start 197.88 131.98) (end 197.88 142.14) (width 0.25) (layer "F.Cu") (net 3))
 (segment (start 157.758618 119.216422) (end 156.769017 120.206023) (width 0.25) (layer "F.Cu") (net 3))
 (segment (start 110.345 118.105) (end 111.52 119.28) (width 0.25) (layer "F.Cu") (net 3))
 (segment (start 197.88 131.98) (end 197.88 124.36) (width 0.25) (layer "F.Cu") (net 3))
 (segment (start 200.42 119.28) (end 195.34 114.2) (width 0.25) (layer "F.Cu") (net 3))
 (segment (start 199.055 107.755) (end 197.88 106.58) (width 0.25) (layer "F.Cu") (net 3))
 (segment (start 169.94 123.65) (end 167.527804 123.65) (width 0.25) (layer "F.Cu") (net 3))
 (segment (start 200.42 121.82) (end 200.42 119.28) (width 0.25) (layer "F.Cu") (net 3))
 (segment (start 180.1 134.52) (end 167.4 134.52) (width 0.25) (layer "F.Cu") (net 3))
 (segment (start 157.758618 112.838618) (end 155 110.08) (width 0.25) (layer "F.Cu") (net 3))
 (segment (start 152.16 131.98) (end 149.62 131.98) (width 0.25) (layer "F.Cu") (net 3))
 (segment (start 197.88 124.36) (end 200.42 121.82) (width 0.25) (layer "F.Cu") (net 3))
 (segment (start 201.785 107.755) (end 199.055 107.755) (width 0.25) (layer "F.Cu") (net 3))
 (segment (start 107.615 118.105) (end 110.345 118.105) (width 0.25) (layer "F.Cu") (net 3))
 (segment (start 153.24822 120.206023) (end 152.258619 119.216422) (width 0.25) (layer "F.Cu") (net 3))
 (segment (start 202.96 106.58) (end 201.785 107.755) (width 0.25) (layer "F.Cu") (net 3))
 (segment (start 157.758618 119.216422) (end 157.758618 112.838618) (width 0.25) (layer "F.Cu") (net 3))
 (segment (start 167.4 134.52) (end 164.86 131.98) (width 0.25) (layer "F.Cu") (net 3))
 (segment (start 167.527804 123.65) (end 164.86 126.317804) (width 0.25) (layer "F.Cu") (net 3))
 (segment (start 149.62 131.98) (end 136.92 144.68) (width 0.25) (layer "F.Cu") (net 3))
 (segment (start 201.785 138.425) (end 201.785 130.615) (width 0.25) (layer "B.Cu") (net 6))
 (segment (start 201.785 130.615) (end 205.5 126.9) (width 0.25) (layer "B.Cu") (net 6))
 (segment (start 208.04 126.9) (end 208.04 101.5) (width 0.25) (layer "B.Cu") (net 6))
 (segment (start 152.16 101.5) (end 142 111.66) (width 0.25) (layer "B.Cu") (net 6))
 (segment (start 202.96 142.14) (end 202.96 139.6) (width 0.25) (layer "B.Cu") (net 6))
 (segment (start 205.5 126.9) (end 208.04 126.9) (width 0.25) (layer "B.Cu") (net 6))
 (segment (start 208.04 101.5) (end 152.16 101.5) (width 0.25) (layer "B.Cu") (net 6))
 (segment (start 202.96 139.6) (end 201.785 138.425) (width 0.25) (layer "B.Cu") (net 6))
 (segment (start 142 111.66) (end 136.92 111.66) (width 0.25) (layer "B.Cu") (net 6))
 (segment (start 134.38 101.5) (end 114.06 101.5) (width 0.25) (layer "F.Cu") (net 4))
 (segment (start 134.38 111.66) (end 134.38 101.5) (width 0.25) (layer "F.Cu") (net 4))
 (segment (start 114.06 101.5) (end 111.52 104.04) (width 0.25) (layer "F.Cu") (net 4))
 (segment (start 136.92 114.2) (end 134.38 111.66) (width 0.25) (layer "F.Cu") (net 4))
 (segment (start 124.22 104.04) (end 136.92 116.74) (width 0.25) (layer "F.Cu") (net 5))
 (segment (start 114.06 104.04) (end 124.22 104.04) (width 0.25) (layer "F.Cu") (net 5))
 (segment (start 142 114.2) (end 136.92 119.28) (width 0.25) (layer "F.Cu") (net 7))
 (segment (start 142 111.66) (end 142 114.2) (width 0.25) (layer "F.Cu") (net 7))
 (segment (start 152.16 101.5) (end 142 111.66) (width 0.25) (layer "F.Cu") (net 7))
 (segment (start 205.5 142.14) (end 208.04 142.14) (width 0.25) (layer "F.Cu") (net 7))
 (segment (start 208.04 142.14) (end 208.04 101.5) (width 0.25) (layer "F.Cu") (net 7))
 (segment (start 208.04 101.5) (end 152.16 101.5) (width 0.25) (layer "F.Cu") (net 7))
 (segment (start 187.72 121.105) (end 192.085 121.105) (width 0.25) (layer "F.Cu") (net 26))
 (segment (start 192.085 121.105) (end 192.8 121.82) (width 0.25) (layer "F.Cu") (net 26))
 (via blind (at 192.8 121.82) (size 0.8) (drill 0.4) (layers "F.Cu" "B.Cu") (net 26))
 (segment (start 153.332919 122.201412) (end 152.703609 122.830722) (width 0.25) (layer "B.Cu") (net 26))
 (segment (start 195.34 121.82) (end 192.8 121.82) (width 0.25) (layer "B.Cu") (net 26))
 (segment (start 143.010722 122.830722) (end 142 121.82) (width 0.25) (layer "B.Cu") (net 26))
 (segment (start 142 121.82) (end 136.92 121.82) (width 0.25) (layer "B.Cu") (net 26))
 (segment (start 154.422457 120.682122) (end 153.332919 121.77166) (width 0.25) (layer "B.Cu") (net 26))
 (segment (start 152.703609 122.830722) (end 143.010722 122.830722) (width 0.25) (layer "B.Cu") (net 26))
 (segment (start 192.8 121.82) (end 191.662122 120.682122) (width 0.25) (layer "B.Cu") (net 26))
 (segment (start 191.662122 120.682122) (end 154.422457 120.682122) (width 0.25) (layer "B.Cu") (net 26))
 (segment (start 202.96 114.2) (end 195.34 121.82) (width 0.25) (layer "B.Cu") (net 26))
 (segment (start 153.332919 121.77166) (end 153.332919 122.201412) (width 0.25) (layer "B.Cu") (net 26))
 (segment (start 141.0875 123.4475) (end 142 124.36) (width 0.25) (layer "B.Cu") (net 30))
 (segment (start 157.758618 121.926881) (end 157.758618 121.756422) (width 0.25) (layer "B.Cu") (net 30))
 (segment (start 137.8325 123.4475) (end 136.92 124.36) (width 0.25) (layer "B.Cu") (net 30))
 (segment (start 141.0875 123.4475) (end 137.8325 123.4475) (width 0.25) (layer "B.Cu") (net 30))
 (segment (start 155.325499 124.36) (end 157.758618 121.926881) (width 0.25) (layer "B.Cu") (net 30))
 (segment (start 142 124.36) (end 155.325499 124.36) (width 0.25) (layer "B.Cu") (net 30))
 (segment (start 131.84 127.8125) (end 131.5775 128.075) (width 0.25) (layer "B.Cu") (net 9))
 (segment (start 132.7525 126.9) (end 131.84 127.8125) (width 0.25) (layer "B.Cu") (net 9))
 (segment (start 120.315 128.075) (end 114.06 121.82) (width 0.25) (layer "B.Cu") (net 9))
 (segment (start 114.06 121.82) (end 114.06 119.28) (width 0.25) (layer "B.Cu") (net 9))
 (segment (start 131.5775 128.075) (end 120.315 128.075) (width 0.25) (layer "B.Cu") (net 9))
 (segment (start 136.92 126.9) (end 132.7525 126.9) (width 0.25) (layer "B.Cu") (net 9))
 (segment (start 150.54 107.54) (end 152.46 107.54) (width 0.25) (layer "F.Cu") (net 27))
 (segment (start 143.6275 128.5275) (end 143.6275 114.4525) (width 0.25) (layer "F.Cu") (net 27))
 (segment (start 139.46 129.44) (end 136.92 129.44) (width 0.25) (layer "F.Cu") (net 27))
 (segment (start 140.3725 128.5275) (end 139.46 129.44) (width 0.25) (layer "F.Cu") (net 27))
 (segment (start 143.6275 114.4525) (end 150.54 107.54) (width 0.25) (layer "F.Cu") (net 27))
 (segment (start 143.6275 128.5275) (end 140.3725 128.5275) (width 0.25) (layer "F.Cu") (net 27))
 (segment (start 197.88 114.2) (end 192.8 109.12) (width 0.25) (layer "F.Cu") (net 13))
 (segment (start 192.8 109.12) (end 180.1 109.12) (width 0.25) (layer "F.Cu") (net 13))
 (segment (start 152.258619 125.888881) (end 152.16 125.9875) (width 0.25) (layer "F.Cu") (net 2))
 (segment (start 152.258619 121.756422) (end 152.258619 125.888881) (width 0.25) (layer "F.Cu") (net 2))
 (segment (start 112.885 113.025) (end 111.52 111.66) (width 0.25) (layer "F.Cu") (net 25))
 (segment (start 125.9225 127.5951) (end 125.9225 116.780799) (width 0.25) (layer "F.Cu") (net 25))
 (segment (start 122.166701 113.025) (end 112.885 113.025) (width 0.25) (layer "F.Cu") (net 25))
 (segment (start 130.3074 131.98) (end 125.9225 127.5951) (width 0.25) (layer "F.Cu") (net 25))
 (segment (start 125.9225 116.780799) (end 122.166701 113.025) (width 0.25) (layer "F.Cu") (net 25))
 (segment (start 136.92 131.98) (end 130.3074 131.98) (width 0.25) (layer "F.Cu") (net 25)))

